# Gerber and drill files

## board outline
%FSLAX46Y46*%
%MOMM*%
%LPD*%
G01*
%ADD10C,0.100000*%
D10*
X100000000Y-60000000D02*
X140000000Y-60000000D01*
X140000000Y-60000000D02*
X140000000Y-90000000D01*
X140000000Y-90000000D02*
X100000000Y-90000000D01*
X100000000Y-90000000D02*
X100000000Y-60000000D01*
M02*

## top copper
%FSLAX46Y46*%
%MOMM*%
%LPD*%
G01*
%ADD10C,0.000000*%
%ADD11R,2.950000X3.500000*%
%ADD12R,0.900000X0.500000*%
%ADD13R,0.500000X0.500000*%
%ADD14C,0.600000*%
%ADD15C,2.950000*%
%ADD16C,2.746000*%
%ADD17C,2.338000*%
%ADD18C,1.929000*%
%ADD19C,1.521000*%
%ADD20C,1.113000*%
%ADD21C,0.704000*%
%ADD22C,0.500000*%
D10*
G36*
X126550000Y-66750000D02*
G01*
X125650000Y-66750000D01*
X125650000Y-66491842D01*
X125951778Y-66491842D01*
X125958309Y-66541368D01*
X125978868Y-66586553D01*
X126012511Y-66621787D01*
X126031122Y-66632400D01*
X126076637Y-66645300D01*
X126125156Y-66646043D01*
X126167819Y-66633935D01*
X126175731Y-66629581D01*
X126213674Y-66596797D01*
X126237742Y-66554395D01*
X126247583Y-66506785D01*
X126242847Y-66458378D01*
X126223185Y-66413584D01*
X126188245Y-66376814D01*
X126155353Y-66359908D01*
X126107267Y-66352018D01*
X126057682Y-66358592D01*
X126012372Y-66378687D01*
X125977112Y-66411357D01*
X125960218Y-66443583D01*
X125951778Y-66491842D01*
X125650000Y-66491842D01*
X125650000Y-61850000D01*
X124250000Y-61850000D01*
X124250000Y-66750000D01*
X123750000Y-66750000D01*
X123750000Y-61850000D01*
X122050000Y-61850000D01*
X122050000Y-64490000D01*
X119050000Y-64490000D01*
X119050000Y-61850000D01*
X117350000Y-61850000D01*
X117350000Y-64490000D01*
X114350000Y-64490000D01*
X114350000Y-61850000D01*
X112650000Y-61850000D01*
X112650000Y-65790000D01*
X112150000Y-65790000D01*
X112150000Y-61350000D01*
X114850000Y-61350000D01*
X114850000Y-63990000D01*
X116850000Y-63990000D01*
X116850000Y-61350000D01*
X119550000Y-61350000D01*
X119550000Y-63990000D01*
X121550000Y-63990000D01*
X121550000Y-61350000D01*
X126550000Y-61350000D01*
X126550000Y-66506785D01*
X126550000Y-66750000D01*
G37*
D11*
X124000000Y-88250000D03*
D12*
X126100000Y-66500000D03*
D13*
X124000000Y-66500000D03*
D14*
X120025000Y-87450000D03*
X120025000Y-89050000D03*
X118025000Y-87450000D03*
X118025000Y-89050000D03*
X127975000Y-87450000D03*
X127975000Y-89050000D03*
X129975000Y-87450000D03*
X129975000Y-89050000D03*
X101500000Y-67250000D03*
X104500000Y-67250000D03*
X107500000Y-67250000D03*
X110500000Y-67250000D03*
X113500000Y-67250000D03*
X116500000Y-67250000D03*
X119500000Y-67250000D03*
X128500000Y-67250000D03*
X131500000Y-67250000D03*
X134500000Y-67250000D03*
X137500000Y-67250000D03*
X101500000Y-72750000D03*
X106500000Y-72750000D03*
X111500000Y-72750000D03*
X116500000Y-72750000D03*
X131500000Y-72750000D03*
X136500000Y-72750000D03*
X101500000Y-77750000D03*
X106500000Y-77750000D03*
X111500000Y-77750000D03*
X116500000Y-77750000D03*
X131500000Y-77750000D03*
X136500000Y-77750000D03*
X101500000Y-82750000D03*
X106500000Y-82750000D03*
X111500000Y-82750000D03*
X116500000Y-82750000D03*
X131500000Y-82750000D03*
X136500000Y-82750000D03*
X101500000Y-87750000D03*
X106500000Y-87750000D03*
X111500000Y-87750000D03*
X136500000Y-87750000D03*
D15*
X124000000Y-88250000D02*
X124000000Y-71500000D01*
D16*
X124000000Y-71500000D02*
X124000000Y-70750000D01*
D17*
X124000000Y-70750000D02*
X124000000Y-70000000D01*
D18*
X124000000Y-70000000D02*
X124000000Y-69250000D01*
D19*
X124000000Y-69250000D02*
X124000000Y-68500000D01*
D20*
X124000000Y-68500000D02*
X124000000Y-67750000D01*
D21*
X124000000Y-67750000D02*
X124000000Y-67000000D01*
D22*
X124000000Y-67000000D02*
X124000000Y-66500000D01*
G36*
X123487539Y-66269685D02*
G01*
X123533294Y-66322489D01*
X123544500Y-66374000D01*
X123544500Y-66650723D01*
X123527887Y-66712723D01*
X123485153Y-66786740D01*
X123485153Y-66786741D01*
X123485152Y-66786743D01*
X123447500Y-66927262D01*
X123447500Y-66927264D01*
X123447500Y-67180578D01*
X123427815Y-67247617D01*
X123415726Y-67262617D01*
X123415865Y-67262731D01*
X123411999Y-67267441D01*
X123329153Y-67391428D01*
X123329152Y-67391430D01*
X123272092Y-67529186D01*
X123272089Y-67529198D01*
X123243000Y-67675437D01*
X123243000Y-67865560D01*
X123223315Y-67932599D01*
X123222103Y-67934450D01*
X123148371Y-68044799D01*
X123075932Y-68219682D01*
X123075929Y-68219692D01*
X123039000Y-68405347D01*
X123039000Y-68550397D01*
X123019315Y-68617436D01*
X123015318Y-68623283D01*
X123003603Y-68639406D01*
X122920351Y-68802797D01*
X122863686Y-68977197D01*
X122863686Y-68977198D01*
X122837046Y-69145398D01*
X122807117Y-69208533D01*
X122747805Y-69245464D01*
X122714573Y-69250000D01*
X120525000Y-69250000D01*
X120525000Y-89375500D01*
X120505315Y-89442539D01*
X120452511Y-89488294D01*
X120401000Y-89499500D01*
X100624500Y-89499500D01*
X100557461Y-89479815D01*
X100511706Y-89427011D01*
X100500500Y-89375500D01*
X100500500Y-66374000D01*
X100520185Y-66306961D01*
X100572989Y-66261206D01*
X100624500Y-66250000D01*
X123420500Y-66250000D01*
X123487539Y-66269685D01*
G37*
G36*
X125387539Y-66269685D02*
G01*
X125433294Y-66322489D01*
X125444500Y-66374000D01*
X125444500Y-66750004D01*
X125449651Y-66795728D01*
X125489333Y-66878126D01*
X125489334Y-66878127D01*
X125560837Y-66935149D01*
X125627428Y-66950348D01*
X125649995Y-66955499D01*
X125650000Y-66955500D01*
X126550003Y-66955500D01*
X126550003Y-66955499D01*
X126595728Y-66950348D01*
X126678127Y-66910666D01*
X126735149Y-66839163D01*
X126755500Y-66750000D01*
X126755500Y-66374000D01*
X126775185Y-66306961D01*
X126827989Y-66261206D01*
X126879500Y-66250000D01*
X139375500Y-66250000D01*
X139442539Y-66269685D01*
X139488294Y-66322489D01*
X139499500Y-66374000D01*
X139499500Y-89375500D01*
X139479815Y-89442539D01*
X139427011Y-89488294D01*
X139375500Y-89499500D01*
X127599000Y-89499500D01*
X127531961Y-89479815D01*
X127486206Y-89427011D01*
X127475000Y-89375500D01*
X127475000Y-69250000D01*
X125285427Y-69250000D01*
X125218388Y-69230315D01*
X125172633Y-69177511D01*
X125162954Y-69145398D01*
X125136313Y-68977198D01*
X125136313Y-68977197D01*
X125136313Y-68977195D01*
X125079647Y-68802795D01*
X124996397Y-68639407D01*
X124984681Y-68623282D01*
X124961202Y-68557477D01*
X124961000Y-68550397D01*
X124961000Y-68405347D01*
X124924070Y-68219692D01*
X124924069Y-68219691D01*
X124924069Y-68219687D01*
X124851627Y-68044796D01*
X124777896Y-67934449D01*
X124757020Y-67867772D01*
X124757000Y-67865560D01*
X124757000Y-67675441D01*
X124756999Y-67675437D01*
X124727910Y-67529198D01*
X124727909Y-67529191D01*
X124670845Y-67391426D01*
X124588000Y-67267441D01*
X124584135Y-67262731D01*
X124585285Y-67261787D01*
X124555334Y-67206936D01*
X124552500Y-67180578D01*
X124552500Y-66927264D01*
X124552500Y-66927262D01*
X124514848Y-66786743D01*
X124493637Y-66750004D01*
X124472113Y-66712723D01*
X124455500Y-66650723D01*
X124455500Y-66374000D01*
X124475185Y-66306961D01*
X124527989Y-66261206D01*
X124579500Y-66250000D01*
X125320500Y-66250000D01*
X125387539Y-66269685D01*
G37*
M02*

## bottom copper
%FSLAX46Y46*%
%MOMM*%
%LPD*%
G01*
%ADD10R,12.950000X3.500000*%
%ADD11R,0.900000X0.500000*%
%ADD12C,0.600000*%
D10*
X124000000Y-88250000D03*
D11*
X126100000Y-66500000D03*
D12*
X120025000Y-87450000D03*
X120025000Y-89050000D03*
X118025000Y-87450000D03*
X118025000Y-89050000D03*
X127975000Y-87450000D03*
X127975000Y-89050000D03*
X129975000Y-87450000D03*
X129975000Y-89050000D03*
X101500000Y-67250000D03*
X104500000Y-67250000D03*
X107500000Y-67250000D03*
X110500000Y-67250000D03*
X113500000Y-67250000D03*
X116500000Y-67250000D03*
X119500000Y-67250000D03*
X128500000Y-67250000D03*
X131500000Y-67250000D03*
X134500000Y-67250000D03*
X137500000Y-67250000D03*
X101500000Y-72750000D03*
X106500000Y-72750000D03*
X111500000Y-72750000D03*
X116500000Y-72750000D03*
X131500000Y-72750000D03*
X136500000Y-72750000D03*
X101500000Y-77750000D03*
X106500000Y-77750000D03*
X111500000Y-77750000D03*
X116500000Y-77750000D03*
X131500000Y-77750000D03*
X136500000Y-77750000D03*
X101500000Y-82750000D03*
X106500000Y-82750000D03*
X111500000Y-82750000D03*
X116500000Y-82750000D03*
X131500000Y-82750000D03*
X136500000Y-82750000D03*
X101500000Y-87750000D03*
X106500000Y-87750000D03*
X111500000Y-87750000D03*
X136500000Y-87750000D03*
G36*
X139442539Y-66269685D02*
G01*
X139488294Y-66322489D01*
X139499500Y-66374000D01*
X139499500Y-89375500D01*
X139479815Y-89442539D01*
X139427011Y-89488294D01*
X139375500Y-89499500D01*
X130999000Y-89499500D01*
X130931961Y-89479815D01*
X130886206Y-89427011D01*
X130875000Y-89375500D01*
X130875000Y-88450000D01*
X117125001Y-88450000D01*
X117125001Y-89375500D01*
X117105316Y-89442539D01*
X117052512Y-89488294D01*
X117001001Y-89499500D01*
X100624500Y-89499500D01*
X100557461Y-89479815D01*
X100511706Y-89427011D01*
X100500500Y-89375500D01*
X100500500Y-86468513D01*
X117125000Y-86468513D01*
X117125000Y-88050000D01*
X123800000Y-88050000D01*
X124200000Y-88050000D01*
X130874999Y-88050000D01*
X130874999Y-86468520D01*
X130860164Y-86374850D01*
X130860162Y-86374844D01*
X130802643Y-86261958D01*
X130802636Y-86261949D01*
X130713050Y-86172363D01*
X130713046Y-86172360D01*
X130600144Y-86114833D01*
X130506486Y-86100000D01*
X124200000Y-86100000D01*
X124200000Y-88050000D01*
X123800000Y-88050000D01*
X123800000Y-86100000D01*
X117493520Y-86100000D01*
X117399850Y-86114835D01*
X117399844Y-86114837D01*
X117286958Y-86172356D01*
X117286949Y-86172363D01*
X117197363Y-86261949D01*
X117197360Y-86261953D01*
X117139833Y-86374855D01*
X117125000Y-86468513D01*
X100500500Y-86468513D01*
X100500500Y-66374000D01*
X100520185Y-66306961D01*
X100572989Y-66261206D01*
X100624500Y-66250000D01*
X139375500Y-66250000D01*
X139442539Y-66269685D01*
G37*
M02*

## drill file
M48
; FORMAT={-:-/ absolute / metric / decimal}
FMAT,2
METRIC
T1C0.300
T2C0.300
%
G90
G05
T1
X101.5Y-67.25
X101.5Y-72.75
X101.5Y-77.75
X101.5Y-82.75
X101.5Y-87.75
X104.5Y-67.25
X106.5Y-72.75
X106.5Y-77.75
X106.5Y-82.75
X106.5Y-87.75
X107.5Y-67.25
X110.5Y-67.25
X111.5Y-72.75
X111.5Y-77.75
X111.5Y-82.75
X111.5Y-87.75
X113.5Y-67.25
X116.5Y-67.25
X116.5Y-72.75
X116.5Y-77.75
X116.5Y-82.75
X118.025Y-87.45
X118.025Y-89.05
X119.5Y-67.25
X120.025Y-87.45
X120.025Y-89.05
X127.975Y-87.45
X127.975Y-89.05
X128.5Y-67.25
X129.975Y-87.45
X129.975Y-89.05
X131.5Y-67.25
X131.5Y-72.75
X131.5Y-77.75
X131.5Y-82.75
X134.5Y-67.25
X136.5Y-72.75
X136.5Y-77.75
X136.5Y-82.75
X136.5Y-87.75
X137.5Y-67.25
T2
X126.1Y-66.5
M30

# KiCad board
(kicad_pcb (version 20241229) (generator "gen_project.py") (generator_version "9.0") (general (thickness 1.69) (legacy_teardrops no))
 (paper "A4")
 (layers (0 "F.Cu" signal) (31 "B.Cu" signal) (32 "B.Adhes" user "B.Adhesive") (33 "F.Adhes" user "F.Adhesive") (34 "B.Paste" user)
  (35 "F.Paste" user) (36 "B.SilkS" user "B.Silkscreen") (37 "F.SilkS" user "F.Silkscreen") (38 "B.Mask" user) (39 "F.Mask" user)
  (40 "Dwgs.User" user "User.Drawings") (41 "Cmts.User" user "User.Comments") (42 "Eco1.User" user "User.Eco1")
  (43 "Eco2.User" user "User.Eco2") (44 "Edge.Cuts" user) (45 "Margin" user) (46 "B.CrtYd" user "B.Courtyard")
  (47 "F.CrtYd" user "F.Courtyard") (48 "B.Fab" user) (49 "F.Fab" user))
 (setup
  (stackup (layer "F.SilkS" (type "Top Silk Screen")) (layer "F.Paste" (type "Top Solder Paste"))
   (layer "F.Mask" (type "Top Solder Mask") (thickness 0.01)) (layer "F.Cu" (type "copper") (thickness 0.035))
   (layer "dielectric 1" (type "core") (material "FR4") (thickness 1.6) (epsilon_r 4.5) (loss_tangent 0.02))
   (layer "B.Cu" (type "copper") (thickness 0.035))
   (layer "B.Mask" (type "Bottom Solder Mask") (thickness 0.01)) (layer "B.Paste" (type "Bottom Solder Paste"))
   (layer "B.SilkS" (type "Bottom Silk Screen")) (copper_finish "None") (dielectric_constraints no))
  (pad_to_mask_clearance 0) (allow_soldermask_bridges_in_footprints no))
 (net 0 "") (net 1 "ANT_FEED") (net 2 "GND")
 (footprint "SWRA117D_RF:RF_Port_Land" (layer "F.Cu") (at 124 90 90)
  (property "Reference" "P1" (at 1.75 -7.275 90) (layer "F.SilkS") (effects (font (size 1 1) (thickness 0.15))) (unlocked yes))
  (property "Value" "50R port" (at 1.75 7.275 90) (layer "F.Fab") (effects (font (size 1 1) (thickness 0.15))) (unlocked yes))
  (pad "1" smd rect (at 1.75 0 90) (size 3.5 2.95) (layers "F.Cu" "F.Paste" "F.Mask") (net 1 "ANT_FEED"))
  (pad "2" smd rect (at 1.75 0 90) (size 3.5 12.95) (layers "B.Cu" "B.Mask") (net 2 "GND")))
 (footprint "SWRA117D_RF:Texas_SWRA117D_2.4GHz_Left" (layer "F.Cu") (at 124 66.5)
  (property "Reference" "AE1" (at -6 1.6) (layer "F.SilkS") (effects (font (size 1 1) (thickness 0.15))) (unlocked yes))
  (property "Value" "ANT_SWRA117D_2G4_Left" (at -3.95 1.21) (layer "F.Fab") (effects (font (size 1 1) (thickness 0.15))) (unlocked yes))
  (fp_poly
   (pts (xy -2.45 -2.51) (xy -4.45 -2.51) (xy -4.45 -5.15) (xy -7.15 -5.15) (xy -7.15 -2.51) (xy -9.15 -2.51) (xy -9.15 -5.15)
    (xy -11.85 -5.15) (xy -11.85 -0.71) (xy -11.35 -0.71) (xy -11.35 -4.65) (xy -9.65 -4.65) (xy -9.65 -2.01) (xy -6.65 -2.01)
    (xy -6.65 -4.65) (xy -4.95 -4.65) (xy -4.95 -2.01) (xy -1.95 -2.01) (xy -1.95 -4.65) (xy -0.25 -4.65) (xy -0.25 0.25) (xy 0.25 0.25)
    (xy 0.25 -4.65) (xy 1.65 -4.65) (xy 1.65 0.25) (xy 2.55 0.25) (xy 2.55 0.006785) (xy 2.247583 0.006785) (xy 2.237742 0.054395)
    (xy 2.213674 0.096797) (xy 2.175731 0.129581) (xy 2.167819 0.133935) (xy 2.125156 0.146043) (xy 2.076637 0.1453) (xy 2.031122 0.1324)
    (xy 2.012511 0.121787) (xy 1.978868 0.086553) (xy 1.958309 0.041368) (xy 1.951778 -0.008158) (xy 1.960218 -0.056417)
    (xy 1.977112 -0.088643) (xy 2.012372 -0.121313) (xy 2.057682 -0.141408) (xy 2.107267 -0.147982) (xy 2.155353 -0.140092)
    (xy 2.188245 -0.123186) (xy 2.223185 -0.086416) (xy 2.242847 -0.041622) (xy 2.247583 0.006785) (xy 2.55 0.006785) (xy 2.55 -5.15)
    (xy -2.45 -5.15) (xy -2.45 -2.51))
   (stroke (width 0) (type solid)) (fill yes) (layer "F.Cu"))
  (pad "2" thru_hole rect (at 2.1 0) (size 0.9 0.5) (drill 0.3) (layers "*.Cu") (zone_connect 2) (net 2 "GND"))
  (pad "1" smd rect (at 0 0) (size 0.5 0.5) (layers "F.Cu") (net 1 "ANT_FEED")))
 (gr_line (start 100 60) (end 140 60) (stroke (width 0.1) (type solid)) (layer "Edge.Cuts"))
 (gr_line (start 140 60) (end 140 90) (stroke (width 0.1) (type solid)) (layer "Edge.Cuts"))
 (gr_line (start 140 90) (end 100 90) (stroke (width 0.1) (type solid)) (layer "Edge.Cuts"))
 (gr_line (start 100 90) (end 100 60) (stroke (width 0.1) (type solid)) (layer "Edge.Cuts"))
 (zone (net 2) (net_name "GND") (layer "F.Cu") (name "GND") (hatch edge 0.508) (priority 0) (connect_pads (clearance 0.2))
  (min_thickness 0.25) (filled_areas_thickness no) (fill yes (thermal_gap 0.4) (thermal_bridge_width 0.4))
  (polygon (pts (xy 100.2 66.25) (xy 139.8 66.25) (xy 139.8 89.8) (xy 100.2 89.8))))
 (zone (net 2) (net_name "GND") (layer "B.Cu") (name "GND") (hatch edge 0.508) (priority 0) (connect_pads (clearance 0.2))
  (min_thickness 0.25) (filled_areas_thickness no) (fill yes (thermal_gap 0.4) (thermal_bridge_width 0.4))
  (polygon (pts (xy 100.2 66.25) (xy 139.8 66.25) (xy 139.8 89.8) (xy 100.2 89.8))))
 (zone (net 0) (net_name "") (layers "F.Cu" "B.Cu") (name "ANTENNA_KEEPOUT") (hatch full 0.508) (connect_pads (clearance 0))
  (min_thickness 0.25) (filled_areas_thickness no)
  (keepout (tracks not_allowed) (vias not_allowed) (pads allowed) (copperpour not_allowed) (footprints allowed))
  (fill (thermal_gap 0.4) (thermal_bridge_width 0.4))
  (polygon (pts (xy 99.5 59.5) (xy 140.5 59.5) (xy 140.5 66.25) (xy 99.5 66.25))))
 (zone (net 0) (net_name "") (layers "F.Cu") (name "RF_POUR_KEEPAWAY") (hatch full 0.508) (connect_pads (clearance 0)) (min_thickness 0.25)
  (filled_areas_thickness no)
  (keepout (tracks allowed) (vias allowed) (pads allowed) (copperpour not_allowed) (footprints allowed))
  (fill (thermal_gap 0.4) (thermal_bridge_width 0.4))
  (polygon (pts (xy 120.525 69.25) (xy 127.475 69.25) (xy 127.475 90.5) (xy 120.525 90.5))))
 (segment (start 124 88.25) (end 124 71.5) (width 2.95) (layer "F.Cu") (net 1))
 (segment (start 124 71.5) (end 124 70.75) (width 2.746) (layer "F.Cu") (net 1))
 (segment (start 124 70.75) (end 124 70) (width 2.338) (layer "F.Cu") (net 1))
 (segment (start 124 70) (end 124 69.25) (width 1.929) (layer "F.Cu") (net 1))
 (segment (start 124 69.25) (end 124 68.5) (width 1.521) (layer "F.Cu") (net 1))
 (segment (start 124 68.5) (end 124 67.75) (width 1.113) (layer "F.Cu") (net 1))
 (segment (start 124 67.75) (end 124 67) (width 0.704) (layer "F.Cu") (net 1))
 (segment (start 124 67) (end 124 66.5) (width 0.5) (layer "F.Cu") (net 1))
 (via (at 120.025 87.45) (size 0.6) (drill 0.3) (layers "F.Cu" "B.Cu") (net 2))
 (via (at 120.025 89.05) (size 0.6) (drill 0.3) (layers "F.Cu" "B.Cu") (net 2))
 (via (at 118.025 87.45) (size 0.6) (drill 0.3) (layers "F.Cu" "B.Cu") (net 2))
 (via (at 118.025 89.05) (size 0.6) (drill 0.3) (layers "F.Cu" "B.Cu") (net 2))
 (via (at 127.975 87.45) (size 0.6) (drill 0.3) (layers "F.Cu" "B.Cu") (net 2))
 (via (at 127.975 89.05) (size 0.6) (drill 0.3) (layers "F.Cu" "B.Cu") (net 2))
 (via (at 129.975 87.45) (size 0.6) (drill 0.3) (layers "F.Cu" "B.Cu") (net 2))
 (via (at 129.975 89.05) (size 0.6) (drill 0.3) (layers "F.Cu" "B.Cu") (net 2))
 (via (at 101.5 67.25) (size 0.6) (drill 0.3) (layers "F.Cu" "B.Cu") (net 2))
 (via (at 104.5 67.25) (size 0.6) (drill 0.3) (layers "F.Cu" "B.Cu") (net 2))
 (via (at 107.5 67.25) (size 0.6) (drill 0.3) (layers "F.Cu" "B.Cu") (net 2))
 (via (at 110.5 67.25) (size 0.6) (drill 0.3) (layers "F.Cu" "B.Cu") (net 2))
 (via (at 113.5 67.25) (size 0.6) (drill 0.3) (layers "F.Cu" "B.Cu") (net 2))
 (via (at 116.5 67.25) (size 0.6) (drill 0.3) (layers "F.Cu" "B.Cu") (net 2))
 (via (at 119.5 67.25) (size 0.6) (drill 0.3) (layers "F.Cu" "B.Cu") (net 2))
 (via (at 128.5 67.25) (size 0.6) (drill 0.3) (layers "F.Cu" "B.Cu") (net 2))
 (via (at 131.5 67.25) (size 0.6) (drill 0.3) (layers "F.Cu" "B.Cu") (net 2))
 (via (at 134.5 67.25) (size 0.6) (drill 0.3) (layers "F.Cu" "B.Cu") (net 2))
 (via (at 137.5 67.25) (size 0.6) (drill 0.3) (layers "F.Cu" "B.Cu") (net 2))
 (via (at 101.5 72.75) (size 0.6) (drill 0.3) (layers "F.Cu" "B.Cu") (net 2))
 (via (at 106.5 72.75) (size 0.6) (drill 0.3) (layers "F.Cu" "B.Cu") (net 2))
 (via (at 111.5 72.75) (size 0.6) (drill 0.3) (layers "F.Cu" "B.Cu") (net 2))
 (via (at 116.5 72.75) (size 0.6) (drill 0.3) (layers "F.Cu" "B.Cu") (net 2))
 (via (at 131.5 72.75) (size 0.6) (drill 0.3) (layers "F.Cu" "B.Cu") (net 2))
 (via (at 136.5 72.75) (size 0.6) (drill 0.3) (layers "F.Cu" "B.Cu") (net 2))
 (via (at 101.5 77.75) (size 0.6) (drill 0.3) (layers "F.Cu" "B.Cu") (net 2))
 (via (at 106.5 77.75) (size 0.6) (drill 0.3) (layers "F.Cu" "B.Cu") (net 2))
 (via (at 111.5 77.75) (size 0.6) (drill 0.3) (layers "F.Cu" "B.Cu") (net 2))
 (via (at 116.5 77.75) (size 0.6) (drill 0.3) (layers "F.Cu" "B.Cu") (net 2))
 (via (at 131.5 77.75) (size 0.6) (drill 0.3) (layers "F.Cu" "B.Cu") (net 2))
 (via (at 136.5 77.75) (size 0.6) (drill 0.3) (layers "F.Cu" "B.Cu") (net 2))
 (via (at 101.5 82.75) (size 0.6) (drill 0.3) (layers "F.Cu" "B.Cu") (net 2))
 (via (at 106.5 82.75) (size 0.6) (drill 0.3) (layers "F.Cu" "B.Cu") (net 2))
 (via (at 111.5 82.75) (size 0.6) (drill 0.3) (layers "F.Cu" "B.Cu") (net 2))
 (via (at 116.5 82.75) (size 0.6) (drill 0.3) (layers "F.Cu" "B.Cu") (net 2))
 (via (at 131.5 82.75) (size 0.6) (drill 0.3) (layers "F.Cu" "B.Cu") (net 2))
 (via (at 136.5 82.75) (size 0.6) (drill 0.3) (layers "F.Cu" "B.Cu") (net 2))
 (via (at 101.5 87.75) (size 0.6) (drill 0.3) (layers "F.Cu" "B.Cu") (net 2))
 (via (at 106.5 87.75) (size 0.6) (drill 0.3) (layers "F.Cu" "B.Cu") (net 2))
 (via (at 111.5 87.75) (size 0.6) (drill 0.3) (layers "F.Cu" "B.Cu") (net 2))
 (via (at 136.5 87.75) (size 0.6) (drill 0.3) (layers "F.Cu" "B.Cu") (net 2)))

